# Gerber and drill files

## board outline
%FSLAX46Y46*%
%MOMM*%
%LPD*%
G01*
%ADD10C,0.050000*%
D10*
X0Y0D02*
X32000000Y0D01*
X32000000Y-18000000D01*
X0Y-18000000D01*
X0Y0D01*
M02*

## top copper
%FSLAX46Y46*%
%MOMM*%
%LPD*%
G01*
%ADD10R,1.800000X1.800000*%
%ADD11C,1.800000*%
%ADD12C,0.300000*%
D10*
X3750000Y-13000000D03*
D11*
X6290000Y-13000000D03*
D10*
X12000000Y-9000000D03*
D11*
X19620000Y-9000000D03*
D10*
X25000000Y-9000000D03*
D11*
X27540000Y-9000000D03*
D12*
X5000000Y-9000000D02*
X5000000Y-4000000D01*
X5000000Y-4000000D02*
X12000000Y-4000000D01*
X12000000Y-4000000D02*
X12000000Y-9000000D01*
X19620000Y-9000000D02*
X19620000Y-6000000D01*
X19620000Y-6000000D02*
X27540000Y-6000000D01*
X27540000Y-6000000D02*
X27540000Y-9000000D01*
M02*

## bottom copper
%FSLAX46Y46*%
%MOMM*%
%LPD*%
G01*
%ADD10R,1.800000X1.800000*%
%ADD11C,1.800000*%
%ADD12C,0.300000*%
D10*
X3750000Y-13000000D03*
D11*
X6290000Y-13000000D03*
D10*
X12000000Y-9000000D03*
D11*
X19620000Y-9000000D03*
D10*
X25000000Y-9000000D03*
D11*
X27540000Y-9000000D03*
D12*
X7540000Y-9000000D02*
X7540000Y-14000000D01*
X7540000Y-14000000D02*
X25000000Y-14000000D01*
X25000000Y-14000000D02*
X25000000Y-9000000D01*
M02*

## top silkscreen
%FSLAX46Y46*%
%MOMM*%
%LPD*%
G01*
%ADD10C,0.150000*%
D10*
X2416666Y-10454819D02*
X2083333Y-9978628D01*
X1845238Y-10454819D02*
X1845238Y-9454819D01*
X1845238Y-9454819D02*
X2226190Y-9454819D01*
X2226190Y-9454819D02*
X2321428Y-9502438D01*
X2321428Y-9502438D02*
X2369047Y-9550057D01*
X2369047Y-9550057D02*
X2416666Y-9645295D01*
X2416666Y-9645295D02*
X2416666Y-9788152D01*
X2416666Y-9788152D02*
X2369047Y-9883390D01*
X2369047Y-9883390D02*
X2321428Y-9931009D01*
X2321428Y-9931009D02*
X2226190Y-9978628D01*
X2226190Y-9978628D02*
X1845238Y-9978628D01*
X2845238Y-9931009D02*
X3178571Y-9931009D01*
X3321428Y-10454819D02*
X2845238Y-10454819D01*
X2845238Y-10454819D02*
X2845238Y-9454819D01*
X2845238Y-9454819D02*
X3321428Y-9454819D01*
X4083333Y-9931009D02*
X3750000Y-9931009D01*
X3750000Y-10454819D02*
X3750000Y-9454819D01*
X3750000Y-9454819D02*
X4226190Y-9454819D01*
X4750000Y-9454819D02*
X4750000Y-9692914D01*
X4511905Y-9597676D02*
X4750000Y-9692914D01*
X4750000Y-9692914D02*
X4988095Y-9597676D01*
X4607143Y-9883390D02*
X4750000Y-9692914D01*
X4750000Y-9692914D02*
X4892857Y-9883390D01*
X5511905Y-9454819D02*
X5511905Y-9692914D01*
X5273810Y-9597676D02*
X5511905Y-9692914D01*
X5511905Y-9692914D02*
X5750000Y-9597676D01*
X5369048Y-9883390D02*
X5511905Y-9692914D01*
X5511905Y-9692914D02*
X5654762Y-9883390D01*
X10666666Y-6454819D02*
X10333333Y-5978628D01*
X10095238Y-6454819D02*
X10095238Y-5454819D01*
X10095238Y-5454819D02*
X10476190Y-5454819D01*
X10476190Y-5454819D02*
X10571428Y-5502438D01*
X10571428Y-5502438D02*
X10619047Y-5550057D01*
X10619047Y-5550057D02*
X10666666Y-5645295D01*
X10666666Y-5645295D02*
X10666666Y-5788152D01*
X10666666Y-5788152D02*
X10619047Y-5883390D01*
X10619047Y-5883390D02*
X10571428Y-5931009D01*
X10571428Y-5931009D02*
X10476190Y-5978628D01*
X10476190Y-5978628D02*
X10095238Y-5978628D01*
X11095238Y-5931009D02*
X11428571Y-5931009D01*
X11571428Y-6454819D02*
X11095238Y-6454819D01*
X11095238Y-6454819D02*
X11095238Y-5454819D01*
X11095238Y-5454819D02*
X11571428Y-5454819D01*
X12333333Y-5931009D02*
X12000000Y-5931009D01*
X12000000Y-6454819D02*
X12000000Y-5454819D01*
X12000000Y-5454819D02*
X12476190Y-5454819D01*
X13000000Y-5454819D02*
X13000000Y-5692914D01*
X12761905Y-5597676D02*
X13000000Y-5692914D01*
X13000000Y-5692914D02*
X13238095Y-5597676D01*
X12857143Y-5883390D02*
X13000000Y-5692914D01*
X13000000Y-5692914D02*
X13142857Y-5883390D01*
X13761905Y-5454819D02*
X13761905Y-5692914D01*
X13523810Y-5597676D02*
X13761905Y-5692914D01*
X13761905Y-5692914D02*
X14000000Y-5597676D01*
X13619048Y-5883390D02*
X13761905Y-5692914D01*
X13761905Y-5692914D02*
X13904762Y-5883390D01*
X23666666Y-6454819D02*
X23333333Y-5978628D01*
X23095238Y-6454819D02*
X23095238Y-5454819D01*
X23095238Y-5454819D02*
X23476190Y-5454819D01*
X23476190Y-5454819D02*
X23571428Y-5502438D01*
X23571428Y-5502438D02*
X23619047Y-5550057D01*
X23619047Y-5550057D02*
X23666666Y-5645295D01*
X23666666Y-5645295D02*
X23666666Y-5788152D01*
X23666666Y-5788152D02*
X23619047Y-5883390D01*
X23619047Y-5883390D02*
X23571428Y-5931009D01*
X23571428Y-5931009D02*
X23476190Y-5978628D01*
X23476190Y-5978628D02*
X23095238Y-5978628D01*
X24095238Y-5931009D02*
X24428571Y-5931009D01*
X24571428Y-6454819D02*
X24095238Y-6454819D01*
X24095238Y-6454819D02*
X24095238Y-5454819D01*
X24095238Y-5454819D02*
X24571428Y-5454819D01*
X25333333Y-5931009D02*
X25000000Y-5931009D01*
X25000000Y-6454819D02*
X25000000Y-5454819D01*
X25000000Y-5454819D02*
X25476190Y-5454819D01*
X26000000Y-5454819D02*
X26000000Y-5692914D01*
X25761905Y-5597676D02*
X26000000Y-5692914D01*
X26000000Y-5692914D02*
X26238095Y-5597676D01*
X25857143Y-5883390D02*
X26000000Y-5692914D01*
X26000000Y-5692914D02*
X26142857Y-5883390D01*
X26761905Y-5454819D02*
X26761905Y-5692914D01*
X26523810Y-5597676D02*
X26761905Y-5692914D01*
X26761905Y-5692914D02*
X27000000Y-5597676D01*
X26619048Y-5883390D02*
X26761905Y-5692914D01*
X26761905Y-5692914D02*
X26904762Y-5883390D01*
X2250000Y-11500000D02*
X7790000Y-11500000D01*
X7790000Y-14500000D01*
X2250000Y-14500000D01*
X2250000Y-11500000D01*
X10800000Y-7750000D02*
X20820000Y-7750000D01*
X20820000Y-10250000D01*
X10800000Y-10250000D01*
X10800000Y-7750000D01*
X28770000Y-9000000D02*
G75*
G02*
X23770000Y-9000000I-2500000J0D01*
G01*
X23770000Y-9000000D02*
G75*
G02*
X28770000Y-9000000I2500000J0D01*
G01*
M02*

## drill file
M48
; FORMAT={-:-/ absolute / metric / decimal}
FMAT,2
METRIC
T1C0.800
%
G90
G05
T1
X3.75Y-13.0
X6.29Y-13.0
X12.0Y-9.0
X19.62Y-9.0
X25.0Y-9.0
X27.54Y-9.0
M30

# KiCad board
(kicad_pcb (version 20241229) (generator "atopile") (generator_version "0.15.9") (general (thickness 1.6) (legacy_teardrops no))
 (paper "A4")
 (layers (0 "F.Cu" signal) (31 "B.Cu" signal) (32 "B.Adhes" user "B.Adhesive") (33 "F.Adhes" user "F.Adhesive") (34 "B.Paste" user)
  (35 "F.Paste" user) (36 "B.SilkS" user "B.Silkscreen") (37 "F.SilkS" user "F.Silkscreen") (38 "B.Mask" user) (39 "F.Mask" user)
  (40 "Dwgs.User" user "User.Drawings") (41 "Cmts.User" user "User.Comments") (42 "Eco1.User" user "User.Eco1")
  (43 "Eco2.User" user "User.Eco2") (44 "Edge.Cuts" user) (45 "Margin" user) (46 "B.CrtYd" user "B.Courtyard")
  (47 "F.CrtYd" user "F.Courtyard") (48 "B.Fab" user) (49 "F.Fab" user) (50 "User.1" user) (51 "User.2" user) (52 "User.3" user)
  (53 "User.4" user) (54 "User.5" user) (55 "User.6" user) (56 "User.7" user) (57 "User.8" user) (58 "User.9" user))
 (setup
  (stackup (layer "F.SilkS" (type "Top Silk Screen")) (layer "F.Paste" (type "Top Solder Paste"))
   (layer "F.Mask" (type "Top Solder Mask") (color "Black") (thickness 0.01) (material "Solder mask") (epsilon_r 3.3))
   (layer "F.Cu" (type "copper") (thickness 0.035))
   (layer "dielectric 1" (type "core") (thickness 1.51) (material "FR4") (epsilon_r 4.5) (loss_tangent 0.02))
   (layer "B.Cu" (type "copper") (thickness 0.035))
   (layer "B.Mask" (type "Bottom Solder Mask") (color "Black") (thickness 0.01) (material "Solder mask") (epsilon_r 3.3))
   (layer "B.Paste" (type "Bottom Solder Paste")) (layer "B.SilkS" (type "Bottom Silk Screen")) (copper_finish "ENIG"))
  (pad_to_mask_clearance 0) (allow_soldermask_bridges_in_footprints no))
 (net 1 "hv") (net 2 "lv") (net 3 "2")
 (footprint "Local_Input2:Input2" (layer "F.Cu") (at 3.75 13 0)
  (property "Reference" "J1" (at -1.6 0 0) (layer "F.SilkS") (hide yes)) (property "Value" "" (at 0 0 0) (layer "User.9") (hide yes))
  (fp_rect (start -1.5 -1.5) (end 4.04 1.5) (stroke (width 0.15) (type default)) (fill none) (layer "F.SilkS"))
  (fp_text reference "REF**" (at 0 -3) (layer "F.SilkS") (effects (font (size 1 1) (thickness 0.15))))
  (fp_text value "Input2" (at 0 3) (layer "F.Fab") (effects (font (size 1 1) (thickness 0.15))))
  (pad "1" thru_hole rect (at 0 0) (size 1.8 1.8) (drill 0.8) (layers "*.Cu" "*.Mask") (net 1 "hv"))
  (pad "2" thru_hole circle (at 2.54 0) (size 1.8 1.8) (drill 0.8) (layers "*.Cu" "*.Mask") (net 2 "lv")))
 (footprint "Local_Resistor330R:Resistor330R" (layer "F.Cu") (at 12 9 0)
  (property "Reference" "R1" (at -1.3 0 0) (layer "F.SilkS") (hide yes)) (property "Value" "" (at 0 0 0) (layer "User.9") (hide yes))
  (fp_rect (start -1.2 -1.25) (end 8.82 1.25) (stroke (width 0.15) (type default)) (fill none) (layer "F.SilkS"))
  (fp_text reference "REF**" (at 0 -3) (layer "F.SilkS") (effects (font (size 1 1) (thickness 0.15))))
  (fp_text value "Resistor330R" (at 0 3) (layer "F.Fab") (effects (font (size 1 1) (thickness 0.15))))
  (pad "1" thru_hole rect (at 0 0) (size 1.8 1.8) (drill 0.8) (layers "*.Cu" "*.Mask") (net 1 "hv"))
  (pad "2" thru_hole circle (at 7.62 0) (size 1.8 1.8) (drill 0.8) (layers "*.Cu" "*.Mask") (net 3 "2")))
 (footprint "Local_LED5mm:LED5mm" (layer "F.Cu") (at 25 9 0)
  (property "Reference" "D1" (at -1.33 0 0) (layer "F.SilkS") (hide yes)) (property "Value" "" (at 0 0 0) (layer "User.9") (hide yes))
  (fp_circle (center 1.27 0) (end 3.77 0) (stroke (width 0.15) (type default)) (fill none) (layer "F.SilkS"))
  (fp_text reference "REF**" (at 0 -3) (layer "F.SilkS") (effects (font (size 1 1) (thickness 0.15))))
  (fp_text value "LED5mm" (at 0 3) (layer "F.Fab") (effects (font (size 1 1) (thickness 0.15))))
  (pad "1" thru_hole rect (at 0 0) (size 1.8 1.8) (drill 0.8) (layers "*.Cu" "*.Mask") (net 2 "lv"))
  (pad "2" thru_hole circle (at 2.54 0) (size 1.8 1.8) (drill 0.8) (layers "*.Cu" "*.Mask") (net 3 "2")))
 (segment (start 5 9) (end 5 4) (width 0.3) (layer "F.Cu") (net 1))
 (segment (start 5 4) (end 12 4) (width 0.3) (layer "F.Cu") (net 1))
 (segment (start 12 4) (end 12 9) (width 0.3) (layer "F.Cu") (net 1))
 (segment (start 19.62 9) (end 19.62 6) (width 0.3) (layer "F.Cu") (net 3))
 (segment (start 19.62 6) (end 27.54 6) (width 0.3) (layer "F.Cu") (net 3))
 (segment (start 27.54 6) (end 27.54 9) (width 0.3) (layer "F.Cu") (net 3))
 (segment (start 7.54 9) (end 7.54 14) (width 0.3) (layer "B.Cu") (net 2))
 (segment (start 7.54 14) (end 25 14) (width 0.3) (layer "B.Cu") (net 2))
 (segment (start 25 14) (end 25 9) (width 0.3) (layer "B.Cu") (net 2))
 (gr_rect (start 0 0) (end 32 18) (stroke (width 0.05) (type default)) (fill none) (layer "Edge.Cuts")))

